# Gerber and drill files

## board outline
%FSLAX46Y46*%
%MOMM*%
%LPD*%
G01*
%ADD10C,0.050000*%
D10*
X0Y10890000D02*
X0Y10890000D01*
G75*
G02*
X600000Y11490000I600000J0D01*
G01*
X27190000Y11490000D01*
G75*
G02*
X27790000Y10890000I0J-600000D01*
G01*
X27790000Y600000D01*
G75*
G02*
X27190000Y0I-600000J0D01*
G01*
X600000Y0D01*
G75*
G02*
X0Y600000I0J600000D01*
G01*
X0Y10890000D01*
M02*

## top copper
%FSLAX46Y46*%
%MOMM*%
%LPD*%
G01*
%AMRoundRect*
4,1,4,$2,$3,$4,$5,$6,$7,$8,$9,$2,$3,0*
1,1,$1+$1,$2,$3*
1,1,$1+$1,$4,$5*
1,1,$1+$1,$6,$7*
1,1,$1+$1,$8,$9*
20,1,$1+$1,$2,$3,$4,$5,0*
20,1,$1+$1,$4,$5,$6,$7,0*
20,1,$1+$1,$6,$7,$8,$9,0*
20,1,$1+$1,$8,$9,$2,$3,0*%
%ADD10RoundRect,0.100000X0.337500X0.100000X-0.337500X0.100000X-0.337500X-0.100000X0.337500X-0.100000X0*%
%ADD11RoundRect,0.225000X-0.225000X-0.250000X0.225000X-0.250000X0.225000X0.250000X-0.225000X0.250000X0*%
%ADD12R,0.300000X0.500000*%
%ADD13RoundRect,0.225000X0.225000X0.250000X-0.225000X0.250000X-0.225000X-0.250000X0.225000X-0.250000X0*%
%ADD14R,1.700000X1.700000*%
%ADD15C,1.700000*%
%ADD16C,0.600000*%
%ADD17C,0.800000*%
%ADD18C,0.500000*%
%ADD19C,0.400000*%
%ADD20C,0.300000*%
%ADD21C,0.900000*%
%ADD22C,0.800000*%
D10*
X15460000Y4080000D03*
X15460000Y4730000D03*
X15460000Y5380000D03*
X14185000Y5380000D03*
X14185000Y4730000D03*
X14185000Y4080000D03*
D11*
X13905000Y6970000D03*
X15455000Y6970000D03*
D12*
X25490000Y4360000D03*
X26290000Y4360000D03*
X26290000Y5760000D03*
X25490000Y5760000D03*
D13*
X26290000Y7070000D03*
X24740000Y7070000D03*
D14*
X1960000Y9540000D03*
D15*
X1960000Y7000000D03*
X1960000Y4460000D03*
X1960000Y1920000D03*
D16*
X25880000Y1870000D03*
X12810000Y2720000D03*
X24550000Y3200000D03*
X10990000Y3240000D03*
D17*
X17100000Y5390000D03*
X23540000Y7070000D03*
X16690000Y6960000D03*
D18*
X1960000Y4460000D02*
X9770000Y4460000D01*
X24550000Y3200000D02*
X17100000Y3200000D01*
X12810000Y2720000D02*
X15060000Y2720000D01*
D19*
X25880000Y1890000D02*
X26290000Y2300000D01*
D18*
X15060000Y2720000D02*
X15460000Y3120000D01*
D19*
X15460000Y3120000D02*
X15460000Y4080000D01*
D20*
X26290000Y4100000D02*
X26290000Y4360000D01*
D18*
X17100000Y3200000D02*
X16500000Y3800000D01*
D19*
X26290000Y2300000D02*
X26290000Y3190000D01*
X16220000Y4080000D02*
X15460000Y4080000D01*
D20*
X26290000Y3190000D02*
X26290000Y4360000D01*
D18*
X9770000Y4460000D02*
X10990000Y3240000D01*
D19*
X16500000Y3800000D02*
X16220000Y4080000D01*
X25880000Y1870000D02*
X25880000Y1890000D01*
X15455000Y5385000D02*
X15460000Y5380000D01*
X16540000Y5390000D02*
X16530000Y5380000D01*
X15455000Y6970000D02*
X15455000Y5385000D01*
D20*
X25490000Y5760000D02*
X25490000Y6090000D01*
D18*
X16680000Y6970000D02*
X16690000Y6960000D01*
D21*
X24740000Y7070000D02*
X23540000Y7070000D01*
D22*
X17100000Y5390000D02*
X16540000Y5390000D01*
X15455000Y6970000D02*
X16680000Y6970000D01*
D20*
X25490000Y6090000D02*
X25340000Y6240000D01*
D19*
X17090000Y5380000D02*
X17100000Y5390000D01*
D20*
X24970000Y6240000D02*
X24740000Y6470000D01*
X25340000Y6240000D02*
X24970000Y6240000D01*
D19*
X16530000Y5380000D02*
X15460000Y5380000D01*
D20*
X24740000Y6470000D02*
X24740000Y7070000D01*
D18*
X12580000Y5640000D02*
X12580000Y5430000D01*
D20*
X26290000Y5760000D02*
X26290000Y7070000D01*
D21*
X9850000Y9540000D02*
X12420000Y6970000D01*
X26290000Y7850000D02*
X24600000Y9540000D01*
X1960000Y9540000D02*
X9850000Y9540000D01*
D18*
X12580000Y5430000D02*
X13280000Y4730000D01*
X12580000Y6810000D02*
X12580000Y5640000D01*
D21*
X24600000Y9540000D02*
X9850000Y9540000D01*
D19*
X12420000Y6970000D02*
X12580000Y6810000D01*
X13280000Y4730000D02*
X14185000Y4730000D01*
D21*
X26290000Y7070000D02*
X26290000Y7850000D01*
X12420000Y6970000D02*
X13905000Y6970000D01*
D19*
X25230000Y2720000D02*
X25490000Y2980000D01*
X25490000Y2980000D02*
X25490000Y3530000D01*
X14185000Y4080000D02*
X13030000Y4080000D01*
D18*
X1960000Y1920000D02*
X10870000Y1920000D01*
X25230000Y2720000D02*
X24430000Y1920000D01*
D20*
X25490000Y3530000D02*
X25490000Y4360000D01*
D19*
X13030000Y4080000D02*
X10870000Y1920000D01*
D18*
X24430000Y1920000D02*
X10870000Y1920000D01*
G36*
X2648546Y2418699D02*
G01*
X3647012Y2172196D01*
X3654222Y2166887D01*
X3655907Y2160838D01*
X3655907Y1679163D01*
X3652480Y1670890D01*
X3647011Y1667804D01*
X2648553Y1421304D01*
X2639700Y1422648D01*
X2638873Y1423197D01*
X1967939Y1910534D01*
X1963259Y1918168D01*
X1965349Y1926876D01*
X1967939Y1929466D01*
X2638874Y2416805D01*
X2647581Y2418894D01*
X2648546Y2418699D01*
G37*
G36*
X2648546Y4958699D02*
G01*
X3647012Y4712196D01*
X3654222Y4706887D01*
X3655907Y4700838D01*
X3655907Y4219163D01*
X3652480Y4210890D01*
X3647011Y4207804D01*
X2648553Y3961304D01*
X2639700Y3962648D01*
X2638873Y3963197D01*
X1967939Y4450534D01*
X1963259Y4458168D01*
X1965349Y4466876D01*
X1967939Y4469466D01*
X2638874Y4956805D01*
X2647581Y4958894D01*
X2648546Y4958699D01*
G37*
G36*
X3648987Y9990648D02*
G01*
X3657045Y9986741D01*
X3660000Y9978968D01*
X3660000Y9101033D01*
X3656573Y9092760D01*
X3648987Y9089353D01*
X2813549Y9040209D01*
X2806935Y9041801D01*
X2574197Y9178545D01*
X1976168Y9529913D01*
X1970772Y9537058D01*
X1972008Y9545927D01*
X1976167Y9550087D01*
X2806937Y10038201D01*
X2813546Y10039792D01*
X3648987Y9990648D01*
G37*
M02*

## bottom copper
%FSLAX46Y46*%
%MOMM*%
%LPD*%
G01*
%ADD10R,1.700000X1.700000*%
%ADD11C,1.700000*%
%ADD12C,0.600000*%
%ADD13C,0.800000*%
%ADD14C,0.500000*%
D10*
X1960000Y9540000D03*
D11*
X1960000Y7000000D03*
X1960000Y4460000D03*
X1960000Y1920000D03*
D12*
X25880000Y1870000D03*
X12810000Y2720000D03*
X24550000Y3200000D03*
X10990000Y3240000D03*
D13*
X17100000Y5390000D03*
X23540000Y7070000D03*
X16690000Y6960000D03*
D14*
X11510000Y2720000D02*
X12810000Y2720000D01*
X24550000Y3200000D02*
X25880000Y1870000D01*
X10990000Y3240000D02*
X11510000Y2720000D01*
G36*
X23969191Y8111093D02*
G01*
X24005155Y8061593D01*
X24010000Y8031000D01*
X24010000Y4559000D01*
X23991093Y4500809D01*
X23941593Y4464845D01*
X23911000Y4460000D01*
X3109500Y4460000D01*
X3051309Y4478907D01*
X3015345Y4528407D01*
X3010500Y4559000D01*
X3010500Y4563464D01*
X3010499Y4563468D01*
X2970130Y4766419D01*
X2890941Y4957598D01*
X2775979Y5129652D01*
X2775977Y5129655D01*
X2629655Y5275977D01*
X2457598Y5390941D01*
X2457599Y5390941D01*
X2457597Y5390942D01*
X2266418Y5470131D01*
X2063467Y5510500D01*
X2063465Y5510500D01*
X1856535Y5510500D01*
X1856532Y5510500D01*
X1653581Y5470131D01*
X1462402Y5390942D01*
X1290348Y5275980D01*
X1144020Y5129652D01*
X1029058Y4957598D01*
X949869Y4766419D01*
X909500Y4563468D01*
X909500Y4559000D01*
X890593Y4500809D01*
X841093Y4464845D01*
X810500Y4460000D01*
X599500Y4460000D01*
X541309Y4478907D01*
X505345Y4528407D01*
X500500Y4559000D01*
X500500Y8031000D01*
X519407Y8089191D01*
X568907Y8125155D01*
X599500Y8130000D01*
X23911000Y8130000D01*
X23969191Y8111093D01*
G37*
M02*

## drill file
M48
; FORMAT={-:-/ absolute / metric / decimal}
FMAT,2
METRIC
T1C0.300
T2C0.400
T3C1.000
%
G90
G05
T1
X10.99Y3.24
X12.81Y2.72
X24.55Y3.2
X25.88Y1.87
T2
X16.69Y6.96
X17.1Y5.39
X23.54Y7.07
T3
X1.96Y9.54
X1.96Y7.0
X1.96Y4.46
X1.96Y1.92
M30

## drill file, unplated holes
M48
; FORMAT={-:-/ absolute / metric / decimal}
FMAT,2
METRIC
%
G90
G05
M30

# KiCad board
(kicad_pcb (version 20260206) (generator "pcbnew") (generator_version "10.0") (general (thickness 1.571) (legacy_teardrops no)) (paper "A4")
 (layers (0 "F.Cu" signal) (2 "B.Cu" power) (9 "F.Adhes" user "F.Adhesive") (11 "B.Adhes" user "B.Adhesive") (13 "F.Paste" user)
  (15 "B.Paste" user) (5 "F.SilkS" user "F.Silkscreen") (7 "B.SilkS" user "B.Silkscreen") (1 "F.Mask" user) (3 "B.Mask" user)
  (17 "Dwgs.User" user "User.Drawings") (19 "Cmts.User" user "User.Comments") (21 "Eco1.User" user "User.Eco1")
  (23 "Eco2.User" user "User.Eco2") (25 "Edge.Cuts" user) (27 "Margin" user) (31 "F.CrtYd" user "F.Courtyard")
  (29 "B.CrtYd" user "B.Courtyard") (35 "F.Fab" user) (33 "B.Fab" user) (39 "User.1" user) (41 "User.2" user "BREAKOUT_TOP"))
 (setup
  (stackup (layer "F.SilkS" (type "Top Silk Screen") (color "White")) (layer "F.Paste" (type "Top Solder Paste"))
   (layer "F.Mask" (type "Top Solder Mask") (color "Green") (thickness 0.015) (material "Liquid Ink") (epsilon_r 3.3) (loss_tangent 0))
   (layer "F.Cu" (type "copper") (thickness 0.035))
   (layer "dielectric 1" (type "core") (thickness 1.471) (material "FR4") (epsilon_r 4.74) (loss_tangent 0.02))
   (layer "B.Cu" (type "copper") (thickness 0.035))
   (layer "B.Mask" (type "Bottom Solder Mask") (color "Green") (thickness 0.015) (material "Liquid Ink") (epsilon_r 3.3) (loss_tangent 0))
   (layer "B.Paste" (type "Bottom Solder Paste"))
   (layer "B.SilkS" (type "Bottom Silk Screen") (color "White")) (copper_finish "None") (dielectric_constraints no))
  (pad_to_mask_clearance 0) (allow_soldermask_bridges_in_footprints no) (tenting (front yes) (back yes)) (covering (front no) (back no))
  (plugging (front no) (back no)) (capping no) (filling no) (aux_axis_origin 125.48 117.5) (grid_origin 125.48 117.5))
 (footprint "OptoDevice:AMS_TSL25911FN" (layer "F.Cu") (at 140.3025 112.77 180)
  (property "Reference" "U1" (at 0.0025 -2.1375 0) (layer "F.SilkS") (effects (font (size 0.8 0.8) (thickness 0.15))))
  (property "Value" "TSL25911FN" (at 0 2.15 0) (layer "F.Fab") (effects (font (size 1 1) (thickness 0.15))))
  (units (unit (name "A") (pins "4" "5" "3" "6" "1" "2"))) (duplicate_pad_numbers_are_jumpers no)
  (pad "1" smd roundrect (at -0.6375 -0.65 180) (size 0.875 0.4) (layers "F.Cu" "F.Mask" "F.Paste") (roundrect_rratio 0.25) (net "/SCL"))
  (pad "2" smd roundrect (at -0.6375 0 180) (size 0.875 0.4) (layers "F.Cu" "F.Mask" "F.Paste") (roundrect_rratio 0.25)
   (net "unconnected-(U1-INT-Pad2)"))
  (pad "3" smd roundrect (at -0.6375 0.65 180) (size 0.875 0.4) (layers "F.Cu" "F.Mask" "F.Paste") (roundrect_rratio 0.25) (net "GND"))
  (pad "4" smd roundrect (at 0.6375 0.65 180) (size 0.875 0.4) (layers "F.Cu" "F.Mask" "F.Paste") (roundrect_rratio 0.25)
   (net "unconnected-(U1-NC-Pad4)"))
  (pad "5" smd roundrect (at 0.6375 0 180) (size 0.875 0.4) (layers "F.Cu" "F.Mask" "F.Paste") (roundrect_rratio 0.25) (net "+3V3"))
  (pad "6" smd roundrect (at 0.6375 -0.65 180) (size 0.875 0.4) (layers "F.Cu" "F.Mask" "F.Paste") (roundrect_rratio 0.25) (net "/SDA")))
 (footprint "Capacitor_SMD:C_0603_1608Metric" (layer "F.Cu") (at 140.16 110.53)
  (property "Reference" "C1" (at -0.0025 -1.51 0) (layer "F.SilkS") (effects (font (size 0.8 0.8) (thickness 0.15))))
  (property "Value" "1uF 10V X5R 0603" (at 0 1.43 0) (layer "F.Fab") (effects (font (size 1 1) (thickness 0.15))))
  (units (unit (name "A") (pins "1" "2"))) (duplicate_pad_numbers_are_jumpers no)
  (pad "1" smd roundrect (at -0.775 0) (size 0.9 0.95) (layers "F.Cu" "F.Mask" "F.Paste") (roundrect_rratio 0.25) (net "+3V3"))
  (pad "2" smd roundrect (at 0.775 0) (size 0.9 0.95) (layers "F.Cu" "F.Mask" "F.Paste") (roundrect_rratio 0.25) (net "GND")))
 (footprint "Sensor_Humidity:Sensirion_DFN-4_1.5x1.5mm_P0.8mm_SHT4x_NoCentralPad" (layer "F.Cu") (at 151.37 112.44 90)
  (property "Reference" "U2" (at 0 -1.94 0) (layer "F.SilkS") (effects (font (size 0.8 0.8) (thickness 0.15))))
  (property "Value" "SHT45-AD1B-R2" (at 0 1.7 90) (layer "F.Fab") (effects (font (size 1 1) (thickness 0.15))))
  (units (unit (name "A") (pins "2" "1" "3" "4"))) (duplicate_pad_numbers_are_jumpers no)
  (pad "1" smd rect (at -0.7 -0.4 90) (size 0.5 0.3) (layers "F.Cu" "F.Mask" "F.Paste") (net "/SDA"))
  (pad "2" smd rect (at -0.7 0.4 90) (size 0.5 0.3) (layers "F.Cu" "F.Mask" "F.Paste") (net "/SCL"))
  (pad "3" smd rect (at 0.7 0.4 90) (size 0.5 0.3) (layers "F.Cu" "F.Mask" "F.Paste") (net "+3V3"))
  (pad "4" smd rect (at 0.7 -0.4 90) (size 0.5 0.3) (layers "F.Cu" "F.Mask" "F.Paste") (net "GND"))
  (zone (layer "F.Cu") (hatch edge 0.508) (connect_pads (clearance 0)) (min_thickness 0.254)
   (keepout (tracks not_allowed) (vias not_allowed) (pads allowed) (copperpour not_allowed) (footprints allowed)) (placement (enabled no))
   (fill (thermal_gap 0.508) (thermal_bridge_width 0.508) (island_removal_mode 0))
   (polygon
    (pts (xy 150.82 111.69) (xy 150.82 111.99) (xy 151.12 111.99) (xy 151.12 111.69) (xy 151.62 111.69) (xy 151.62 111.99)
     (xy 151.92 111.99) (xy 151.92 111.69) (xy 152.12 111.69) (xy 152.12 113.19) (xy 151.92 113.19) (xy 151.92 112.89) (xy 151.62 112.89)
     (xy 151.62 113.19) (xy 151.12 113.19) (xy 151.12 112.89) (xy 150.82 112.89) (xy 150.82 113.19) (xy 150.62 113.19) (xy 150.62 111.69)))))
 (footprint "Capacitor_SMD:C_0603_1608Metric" (layer "F.Cu") (at 150.995 110.43 180)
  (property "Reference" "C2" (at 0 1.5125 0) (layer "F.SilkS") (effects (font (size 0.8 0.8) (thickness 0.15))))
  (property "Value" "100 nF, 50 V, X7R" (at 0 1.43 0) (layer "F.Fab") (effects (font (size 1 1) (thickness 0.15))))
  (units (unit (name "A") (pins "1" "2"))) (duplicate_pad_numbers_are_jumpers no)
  (pad "1" smd roundrect (at -0.775 0 180) (size 0.9 0.95) (layers "F.Cu" "F.Mask" "F.Paste") (roundrect_rratio 0.25) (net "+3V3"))
  (pad "2" smd roundrect (at 0.775 0 180) (size 0.9 0.95) (layers "F.Cu" "F.Mask" "F.Paste") (roundrect_rratio 0.25) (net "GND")))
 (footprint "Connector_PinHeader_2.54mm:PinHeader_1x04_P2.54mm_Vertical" (layer "B.Cu") (at 127.44 107.96 180)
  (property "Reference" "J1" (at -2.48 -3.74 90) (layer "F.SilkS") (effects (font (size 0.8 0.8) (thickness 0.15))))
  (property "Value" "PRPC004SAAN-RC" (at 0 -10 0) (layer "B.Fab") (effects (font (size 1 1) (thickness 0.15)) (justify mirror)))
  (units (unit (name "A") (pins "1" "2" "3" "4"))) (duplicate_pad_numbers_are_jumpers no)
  (pad "1" thru_hole rect (at 0 0 180) (size 1.7 1.7) (drill 1) (layers "*.Cu" "*.Mask") (remove_unused_layers no) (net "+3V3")
   (teardrops (best_length_ratio 0.5) (max_length 1) (best_width_ratio 1) (max_width 1) (curved_edges no) (filter_ratio 0.9) (enabled yes)
    (allow_two_segments no) (prefer_zone_connections yes)))
  (pad "2" thru_hole circle (at 0 -2.54 180) (size 1.7 1.7) (drill 1) (layers "*.Cu" "*.Mask") (remove_unused_layers no) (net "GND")
   (teardrops (best_length_ratio 0.5) (max_length 1) (best_width_ratio 1) (max_width 1) (curved_edges no) (filter_ratio 0.9) (enabled yes)
    (allow_two_segments no) (prefer_zone_connections yes)))
  (pad "3" thru_hole circle (at 0 -5.08 180) (size 1.7 1.7) (drill 1) (layers "*.Cu" "*.Mask") (remove_unused_layers no) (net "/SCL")
   (teardrops (best_length_ratio 0.5) (max_length 1) (best_width_ratio 1) (max_width 1) (curved_edges no) (filter_ratio 0.9) (enabled yes)
    (allow_two_segments no) (prefer_zone_connections yes)))
  (pad "4" thru_hole circle (at 0 -7.62 180) (size 1.7 1.7) (drill 1) (layers "*.Cu" "*.Mask") (remove_unused_layers no) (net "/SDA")
   (teardrops (best_length_ratio 0.5) (max_length 1) (best_width_ratio 1) (max_width 1) (curved_edges no) (filter_ratio 0.9) (enabled yes)
    (allow_two_segments no) (prefer_zone_connections yes))))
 (gr_rect (start 125.48 106.01) (end 153.27 117.5) (radius 0.6) (stroke (width 0.05) (type solid)) (fill no) (layer "Edge.Cuts"))
 (segment (start 127.44 113.04) (end 135.25 113.04) (width 0.5) (layer "F.Cu") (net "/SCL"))
 (segment (start 150.03 114.3) (end 142.58 114.3) (width 0.5) (layer "F.Cu") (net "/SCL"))
 (segment (start 138.29 114.78) (end 140.54 114.78) (width 0.5) (layer "F.Cu") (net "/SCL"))
 (segment (start 151.36 115.61) (end 151.77 115.2) (width 0.4) (layer "F.Cu") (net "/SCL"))
 (segment (start 140.54 114.78) (end 140.94 114.38) (width 0.5) (layer "F.Cu") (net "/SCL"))
 (segment (start 140.94 114.38) (end 140.94 113.42) (width 0.4) (layer "F.Cu") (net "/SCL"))
 (segment (start 151.77 113.4) (end 151.77 113.14) (width 0.3) (layer "F.Cu") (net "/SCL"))
 (segment (start 142.58 114.3) (end 141.98 113.7) (width 0.5) (layer "F.Cu") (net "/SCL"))
 (segment (start 151.77 115.2) (end 151.77 114.31) (width 0.4) (layer "F.Cu") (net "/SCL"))
 (segment (start 141.7 113.42) (end 140.94 113.42) (width 0.4) (layer "F.Cu") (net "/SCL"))
 (segment (start 151.77 114.31) (end 151.77 113.14) (width 0.3) (layer "F.Cu") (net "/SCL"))
 (segment (start 135.25 113.04) (end 136.47 114.26) (width 0.5) (layer "F.Cu") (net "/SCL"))
 (segment (start 141.98 113.7) (end 141.7 113.42) (width 0.4) (layer "F.Cu") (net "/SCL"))
 (segment (start 151.36 115.63) (end 151.36 115.61) (width 0.4) (layer "F.Cu") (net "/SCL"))
 (via (at 151.36 115.63) (size 0.6) (drill 0.3) (layers "F.Cu" "B.Cu") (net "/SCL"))
 (via (at 138.29 114.78) (size 0.6) (drill 0.3) (layers "F.Cu" "B.Cu") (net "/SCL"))
 (via (at 150.03 114.3) (size 0.6) (drill 0.3) (layers "F.Cu" "B.Cu") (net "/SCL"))
 (via (at 136.47 114.26) (size 0.6) (drill 0.3) (layers "F.Cu" "B.Cu") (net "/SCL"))
 (segment (start 136.99 114.78) (end 138.29 114.78) (width 0.5) (layer "B.Cu") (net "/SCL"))
 (segment (start 150.03 114.3) (end 151.36 115.63) (width 0.5) (layer "B.Cu") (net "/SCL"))
 (segment (start 136.47 114.26) (end 136.99 114.78) (width 0.5) (layer "B.Cu") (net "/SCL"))
 (segment (start 140.935 112.115) (end 140.94 112.12) (width 0.4) (layer "F.Cu") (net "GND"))
 (segment (start 142.02 112.11) (end 142.01 112.12) (width 0.4) (layer "F.Cu") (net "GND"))
 (segment (start 140.935 110.53) (end 140.935 112.115) (width 0.4) (layer "F.Cu") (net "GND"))
 (segment (start 150.97 111.74) (end 150.97 111.41) (width 0.3) (layer "F.Cu") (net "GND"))
 (segment (start 142.16 110.53) (end 142.17 110.54) (width 0.5) (layer "F.Cu") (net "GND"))
 (segment (start 150.22 110.43) (end 149.02 110.43) (width 0.9) (layer "F.Cu") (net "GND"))
 (segment (start 142.58 112.11) (end 142.02 112.11) (width 0.8) (layer "F.Cu") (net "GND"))
 (segment (start 140.935 110.53) (end 142.16 110.53) (width 0.8) (layer "F.Cu") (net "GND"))
 (segment (start 150.97 111.41) (end 150.82 111.26) (width 0.3) (layer "F.Cu") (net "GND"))
 (segment (start 142.57 112.12) (end 142.58 112.11) (width 0.4) (layer "F.Cu") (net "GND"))
 (segment (start 150.45 111.26) (end 150.22 111.03) (width 0.3) (layer "F.Cu") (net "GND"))
 (segment (start 150.82 111.26) (end 150.45 111.26) (width 0.3) (layer "F.Cu") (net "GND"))
 (segment (start 142.01 112.12) (end 140.94 112.12) (width 0.4) (layer "F.Cu") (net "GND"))
 (segment (start 150.22 111.03) (end 150.22 110.43) (width 0.3) (layer "F.Cu") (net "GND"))
 (via (at 142.58 112.11) (size 0.8) (drill 0.4) (layers "F.Cu" "B.Cu") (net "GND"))
 (via (at 149.02 110.43) (size 0.8) (drill 0.4) (layers "F.Cu" "B.Cu") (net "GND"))
 (via (at 142.17 110.54) (size 0.8) (drill 0.4) (layers "F.Cu" "B.Cu") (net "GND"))
 (segment (start 138.06 111.86) (end 138.06 112.07) (width 0.5) (layer "F.Cu") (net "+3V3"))
 (segment (start 151.77 111.74) (end 151.77 110.43) (width 0.3) (layer "F.Cu") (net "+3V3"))
 (segment (start 135.33 107.96) (end 137.9 110.53) (width 0.9) (layer "F.Cu") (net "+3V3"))
 (segment (start 151.77 109.65) (end 150.08 107.96) (width 0.9) (layer "F.Cu") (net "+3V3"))
 (segment (start 127.44 107.96) (end 135.33 107.96) (width 0.9) (layer "F.Cu") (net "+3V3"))
 (segment (start 138.06 112.07) (end 138.76 112.77) (width 0.5) (layer "F.Cu") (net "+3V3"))
 (segment (start 138.06 110.69) (end 138.06 111.86) (width 0.5) (layer "F.Cu") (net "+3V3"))
 (segment (start 150.08 107.96) (end 135.33 107.96) (width 0.9) (layer "F.Cu") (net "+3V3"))
 (segment (start 137.9 110.53) (end 138.06 110.69) (width 0.4) (layer "F.Cu") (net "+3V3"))
 (segment (start 138.76 112.77) (end 139.665 112.77) (width 0.4) (layer "F.Cu") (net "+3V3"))
 (segment (start 151.77 110.43) (end 151.77 109.65) (width 0.9) (layer "F.Cu") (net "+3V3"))
 (segment (start 137.9 110.53) (end 139.385 110.53) (width 0.9) (layer "F.Cu") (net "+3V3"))
 (segment (start 150.71 114.78) (end 150.97 114.52) (width 0.4) (layer "F.Cu") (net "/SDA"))
 (segment (start 150.97 114.52) (end 150.97 113.97) (width 0.4) (layer "F.Cu") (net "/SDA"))
 (segment (start 139.665 113.42) (end 138.51 113.42) (width 0.4) (layer "F.Cu") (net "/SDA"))
 (segment (start 127.44 115.58) (end 136.35 115.58) (width 0.5) (layer "F.Cu") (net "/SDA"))
 (segment (start 150.71 114.78) (end 149.91 115.58) (width 0.5) (layer "F.Cu") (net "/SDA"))
 (segment (start 150.97 113.97) (end 150.97 113.14) (width 0.3) (layer "F.Cu") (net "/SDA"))
 (segment (start 138.51 113.42) (end 136.35 115.58) (width 0.4) (layer "F.Cu") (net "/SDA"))
 (segment (start 149.91 115.58) (end 136.35 115.58) (width 0.5) (layer "F.Cu") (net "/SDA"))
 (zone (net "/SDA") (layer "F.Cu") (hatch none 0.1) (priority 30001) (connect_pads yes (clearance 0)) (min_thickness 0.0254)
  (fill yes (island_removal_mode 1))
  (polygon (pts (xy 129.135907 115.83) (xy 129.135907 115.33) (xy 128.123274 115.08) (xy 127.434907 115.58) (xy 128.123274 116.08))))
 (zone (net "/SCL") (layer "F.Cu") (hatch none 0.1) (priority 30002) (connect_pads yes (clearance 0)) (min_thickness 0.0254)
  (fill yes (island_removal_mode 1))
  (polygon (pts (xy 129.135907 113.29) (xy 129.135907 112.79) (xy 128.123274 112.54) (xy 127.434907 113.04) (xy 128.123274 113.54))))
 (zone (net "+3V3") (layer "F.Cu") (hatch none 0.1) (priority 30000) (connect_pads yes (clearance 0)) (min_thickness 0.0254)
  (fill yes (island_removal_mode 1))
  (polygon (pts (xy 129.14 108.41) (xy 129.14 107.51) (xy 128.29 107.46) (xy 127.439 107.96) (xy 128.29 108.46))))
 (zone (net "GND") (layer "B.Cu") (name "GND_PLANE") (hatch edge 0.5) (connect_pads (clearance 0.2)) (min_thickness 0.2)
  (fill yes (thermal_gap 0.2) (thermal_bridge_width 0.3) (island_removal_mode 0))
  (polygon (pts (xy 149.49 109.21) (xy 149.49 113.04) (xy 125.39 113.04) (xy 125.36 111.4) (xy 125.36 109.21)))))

